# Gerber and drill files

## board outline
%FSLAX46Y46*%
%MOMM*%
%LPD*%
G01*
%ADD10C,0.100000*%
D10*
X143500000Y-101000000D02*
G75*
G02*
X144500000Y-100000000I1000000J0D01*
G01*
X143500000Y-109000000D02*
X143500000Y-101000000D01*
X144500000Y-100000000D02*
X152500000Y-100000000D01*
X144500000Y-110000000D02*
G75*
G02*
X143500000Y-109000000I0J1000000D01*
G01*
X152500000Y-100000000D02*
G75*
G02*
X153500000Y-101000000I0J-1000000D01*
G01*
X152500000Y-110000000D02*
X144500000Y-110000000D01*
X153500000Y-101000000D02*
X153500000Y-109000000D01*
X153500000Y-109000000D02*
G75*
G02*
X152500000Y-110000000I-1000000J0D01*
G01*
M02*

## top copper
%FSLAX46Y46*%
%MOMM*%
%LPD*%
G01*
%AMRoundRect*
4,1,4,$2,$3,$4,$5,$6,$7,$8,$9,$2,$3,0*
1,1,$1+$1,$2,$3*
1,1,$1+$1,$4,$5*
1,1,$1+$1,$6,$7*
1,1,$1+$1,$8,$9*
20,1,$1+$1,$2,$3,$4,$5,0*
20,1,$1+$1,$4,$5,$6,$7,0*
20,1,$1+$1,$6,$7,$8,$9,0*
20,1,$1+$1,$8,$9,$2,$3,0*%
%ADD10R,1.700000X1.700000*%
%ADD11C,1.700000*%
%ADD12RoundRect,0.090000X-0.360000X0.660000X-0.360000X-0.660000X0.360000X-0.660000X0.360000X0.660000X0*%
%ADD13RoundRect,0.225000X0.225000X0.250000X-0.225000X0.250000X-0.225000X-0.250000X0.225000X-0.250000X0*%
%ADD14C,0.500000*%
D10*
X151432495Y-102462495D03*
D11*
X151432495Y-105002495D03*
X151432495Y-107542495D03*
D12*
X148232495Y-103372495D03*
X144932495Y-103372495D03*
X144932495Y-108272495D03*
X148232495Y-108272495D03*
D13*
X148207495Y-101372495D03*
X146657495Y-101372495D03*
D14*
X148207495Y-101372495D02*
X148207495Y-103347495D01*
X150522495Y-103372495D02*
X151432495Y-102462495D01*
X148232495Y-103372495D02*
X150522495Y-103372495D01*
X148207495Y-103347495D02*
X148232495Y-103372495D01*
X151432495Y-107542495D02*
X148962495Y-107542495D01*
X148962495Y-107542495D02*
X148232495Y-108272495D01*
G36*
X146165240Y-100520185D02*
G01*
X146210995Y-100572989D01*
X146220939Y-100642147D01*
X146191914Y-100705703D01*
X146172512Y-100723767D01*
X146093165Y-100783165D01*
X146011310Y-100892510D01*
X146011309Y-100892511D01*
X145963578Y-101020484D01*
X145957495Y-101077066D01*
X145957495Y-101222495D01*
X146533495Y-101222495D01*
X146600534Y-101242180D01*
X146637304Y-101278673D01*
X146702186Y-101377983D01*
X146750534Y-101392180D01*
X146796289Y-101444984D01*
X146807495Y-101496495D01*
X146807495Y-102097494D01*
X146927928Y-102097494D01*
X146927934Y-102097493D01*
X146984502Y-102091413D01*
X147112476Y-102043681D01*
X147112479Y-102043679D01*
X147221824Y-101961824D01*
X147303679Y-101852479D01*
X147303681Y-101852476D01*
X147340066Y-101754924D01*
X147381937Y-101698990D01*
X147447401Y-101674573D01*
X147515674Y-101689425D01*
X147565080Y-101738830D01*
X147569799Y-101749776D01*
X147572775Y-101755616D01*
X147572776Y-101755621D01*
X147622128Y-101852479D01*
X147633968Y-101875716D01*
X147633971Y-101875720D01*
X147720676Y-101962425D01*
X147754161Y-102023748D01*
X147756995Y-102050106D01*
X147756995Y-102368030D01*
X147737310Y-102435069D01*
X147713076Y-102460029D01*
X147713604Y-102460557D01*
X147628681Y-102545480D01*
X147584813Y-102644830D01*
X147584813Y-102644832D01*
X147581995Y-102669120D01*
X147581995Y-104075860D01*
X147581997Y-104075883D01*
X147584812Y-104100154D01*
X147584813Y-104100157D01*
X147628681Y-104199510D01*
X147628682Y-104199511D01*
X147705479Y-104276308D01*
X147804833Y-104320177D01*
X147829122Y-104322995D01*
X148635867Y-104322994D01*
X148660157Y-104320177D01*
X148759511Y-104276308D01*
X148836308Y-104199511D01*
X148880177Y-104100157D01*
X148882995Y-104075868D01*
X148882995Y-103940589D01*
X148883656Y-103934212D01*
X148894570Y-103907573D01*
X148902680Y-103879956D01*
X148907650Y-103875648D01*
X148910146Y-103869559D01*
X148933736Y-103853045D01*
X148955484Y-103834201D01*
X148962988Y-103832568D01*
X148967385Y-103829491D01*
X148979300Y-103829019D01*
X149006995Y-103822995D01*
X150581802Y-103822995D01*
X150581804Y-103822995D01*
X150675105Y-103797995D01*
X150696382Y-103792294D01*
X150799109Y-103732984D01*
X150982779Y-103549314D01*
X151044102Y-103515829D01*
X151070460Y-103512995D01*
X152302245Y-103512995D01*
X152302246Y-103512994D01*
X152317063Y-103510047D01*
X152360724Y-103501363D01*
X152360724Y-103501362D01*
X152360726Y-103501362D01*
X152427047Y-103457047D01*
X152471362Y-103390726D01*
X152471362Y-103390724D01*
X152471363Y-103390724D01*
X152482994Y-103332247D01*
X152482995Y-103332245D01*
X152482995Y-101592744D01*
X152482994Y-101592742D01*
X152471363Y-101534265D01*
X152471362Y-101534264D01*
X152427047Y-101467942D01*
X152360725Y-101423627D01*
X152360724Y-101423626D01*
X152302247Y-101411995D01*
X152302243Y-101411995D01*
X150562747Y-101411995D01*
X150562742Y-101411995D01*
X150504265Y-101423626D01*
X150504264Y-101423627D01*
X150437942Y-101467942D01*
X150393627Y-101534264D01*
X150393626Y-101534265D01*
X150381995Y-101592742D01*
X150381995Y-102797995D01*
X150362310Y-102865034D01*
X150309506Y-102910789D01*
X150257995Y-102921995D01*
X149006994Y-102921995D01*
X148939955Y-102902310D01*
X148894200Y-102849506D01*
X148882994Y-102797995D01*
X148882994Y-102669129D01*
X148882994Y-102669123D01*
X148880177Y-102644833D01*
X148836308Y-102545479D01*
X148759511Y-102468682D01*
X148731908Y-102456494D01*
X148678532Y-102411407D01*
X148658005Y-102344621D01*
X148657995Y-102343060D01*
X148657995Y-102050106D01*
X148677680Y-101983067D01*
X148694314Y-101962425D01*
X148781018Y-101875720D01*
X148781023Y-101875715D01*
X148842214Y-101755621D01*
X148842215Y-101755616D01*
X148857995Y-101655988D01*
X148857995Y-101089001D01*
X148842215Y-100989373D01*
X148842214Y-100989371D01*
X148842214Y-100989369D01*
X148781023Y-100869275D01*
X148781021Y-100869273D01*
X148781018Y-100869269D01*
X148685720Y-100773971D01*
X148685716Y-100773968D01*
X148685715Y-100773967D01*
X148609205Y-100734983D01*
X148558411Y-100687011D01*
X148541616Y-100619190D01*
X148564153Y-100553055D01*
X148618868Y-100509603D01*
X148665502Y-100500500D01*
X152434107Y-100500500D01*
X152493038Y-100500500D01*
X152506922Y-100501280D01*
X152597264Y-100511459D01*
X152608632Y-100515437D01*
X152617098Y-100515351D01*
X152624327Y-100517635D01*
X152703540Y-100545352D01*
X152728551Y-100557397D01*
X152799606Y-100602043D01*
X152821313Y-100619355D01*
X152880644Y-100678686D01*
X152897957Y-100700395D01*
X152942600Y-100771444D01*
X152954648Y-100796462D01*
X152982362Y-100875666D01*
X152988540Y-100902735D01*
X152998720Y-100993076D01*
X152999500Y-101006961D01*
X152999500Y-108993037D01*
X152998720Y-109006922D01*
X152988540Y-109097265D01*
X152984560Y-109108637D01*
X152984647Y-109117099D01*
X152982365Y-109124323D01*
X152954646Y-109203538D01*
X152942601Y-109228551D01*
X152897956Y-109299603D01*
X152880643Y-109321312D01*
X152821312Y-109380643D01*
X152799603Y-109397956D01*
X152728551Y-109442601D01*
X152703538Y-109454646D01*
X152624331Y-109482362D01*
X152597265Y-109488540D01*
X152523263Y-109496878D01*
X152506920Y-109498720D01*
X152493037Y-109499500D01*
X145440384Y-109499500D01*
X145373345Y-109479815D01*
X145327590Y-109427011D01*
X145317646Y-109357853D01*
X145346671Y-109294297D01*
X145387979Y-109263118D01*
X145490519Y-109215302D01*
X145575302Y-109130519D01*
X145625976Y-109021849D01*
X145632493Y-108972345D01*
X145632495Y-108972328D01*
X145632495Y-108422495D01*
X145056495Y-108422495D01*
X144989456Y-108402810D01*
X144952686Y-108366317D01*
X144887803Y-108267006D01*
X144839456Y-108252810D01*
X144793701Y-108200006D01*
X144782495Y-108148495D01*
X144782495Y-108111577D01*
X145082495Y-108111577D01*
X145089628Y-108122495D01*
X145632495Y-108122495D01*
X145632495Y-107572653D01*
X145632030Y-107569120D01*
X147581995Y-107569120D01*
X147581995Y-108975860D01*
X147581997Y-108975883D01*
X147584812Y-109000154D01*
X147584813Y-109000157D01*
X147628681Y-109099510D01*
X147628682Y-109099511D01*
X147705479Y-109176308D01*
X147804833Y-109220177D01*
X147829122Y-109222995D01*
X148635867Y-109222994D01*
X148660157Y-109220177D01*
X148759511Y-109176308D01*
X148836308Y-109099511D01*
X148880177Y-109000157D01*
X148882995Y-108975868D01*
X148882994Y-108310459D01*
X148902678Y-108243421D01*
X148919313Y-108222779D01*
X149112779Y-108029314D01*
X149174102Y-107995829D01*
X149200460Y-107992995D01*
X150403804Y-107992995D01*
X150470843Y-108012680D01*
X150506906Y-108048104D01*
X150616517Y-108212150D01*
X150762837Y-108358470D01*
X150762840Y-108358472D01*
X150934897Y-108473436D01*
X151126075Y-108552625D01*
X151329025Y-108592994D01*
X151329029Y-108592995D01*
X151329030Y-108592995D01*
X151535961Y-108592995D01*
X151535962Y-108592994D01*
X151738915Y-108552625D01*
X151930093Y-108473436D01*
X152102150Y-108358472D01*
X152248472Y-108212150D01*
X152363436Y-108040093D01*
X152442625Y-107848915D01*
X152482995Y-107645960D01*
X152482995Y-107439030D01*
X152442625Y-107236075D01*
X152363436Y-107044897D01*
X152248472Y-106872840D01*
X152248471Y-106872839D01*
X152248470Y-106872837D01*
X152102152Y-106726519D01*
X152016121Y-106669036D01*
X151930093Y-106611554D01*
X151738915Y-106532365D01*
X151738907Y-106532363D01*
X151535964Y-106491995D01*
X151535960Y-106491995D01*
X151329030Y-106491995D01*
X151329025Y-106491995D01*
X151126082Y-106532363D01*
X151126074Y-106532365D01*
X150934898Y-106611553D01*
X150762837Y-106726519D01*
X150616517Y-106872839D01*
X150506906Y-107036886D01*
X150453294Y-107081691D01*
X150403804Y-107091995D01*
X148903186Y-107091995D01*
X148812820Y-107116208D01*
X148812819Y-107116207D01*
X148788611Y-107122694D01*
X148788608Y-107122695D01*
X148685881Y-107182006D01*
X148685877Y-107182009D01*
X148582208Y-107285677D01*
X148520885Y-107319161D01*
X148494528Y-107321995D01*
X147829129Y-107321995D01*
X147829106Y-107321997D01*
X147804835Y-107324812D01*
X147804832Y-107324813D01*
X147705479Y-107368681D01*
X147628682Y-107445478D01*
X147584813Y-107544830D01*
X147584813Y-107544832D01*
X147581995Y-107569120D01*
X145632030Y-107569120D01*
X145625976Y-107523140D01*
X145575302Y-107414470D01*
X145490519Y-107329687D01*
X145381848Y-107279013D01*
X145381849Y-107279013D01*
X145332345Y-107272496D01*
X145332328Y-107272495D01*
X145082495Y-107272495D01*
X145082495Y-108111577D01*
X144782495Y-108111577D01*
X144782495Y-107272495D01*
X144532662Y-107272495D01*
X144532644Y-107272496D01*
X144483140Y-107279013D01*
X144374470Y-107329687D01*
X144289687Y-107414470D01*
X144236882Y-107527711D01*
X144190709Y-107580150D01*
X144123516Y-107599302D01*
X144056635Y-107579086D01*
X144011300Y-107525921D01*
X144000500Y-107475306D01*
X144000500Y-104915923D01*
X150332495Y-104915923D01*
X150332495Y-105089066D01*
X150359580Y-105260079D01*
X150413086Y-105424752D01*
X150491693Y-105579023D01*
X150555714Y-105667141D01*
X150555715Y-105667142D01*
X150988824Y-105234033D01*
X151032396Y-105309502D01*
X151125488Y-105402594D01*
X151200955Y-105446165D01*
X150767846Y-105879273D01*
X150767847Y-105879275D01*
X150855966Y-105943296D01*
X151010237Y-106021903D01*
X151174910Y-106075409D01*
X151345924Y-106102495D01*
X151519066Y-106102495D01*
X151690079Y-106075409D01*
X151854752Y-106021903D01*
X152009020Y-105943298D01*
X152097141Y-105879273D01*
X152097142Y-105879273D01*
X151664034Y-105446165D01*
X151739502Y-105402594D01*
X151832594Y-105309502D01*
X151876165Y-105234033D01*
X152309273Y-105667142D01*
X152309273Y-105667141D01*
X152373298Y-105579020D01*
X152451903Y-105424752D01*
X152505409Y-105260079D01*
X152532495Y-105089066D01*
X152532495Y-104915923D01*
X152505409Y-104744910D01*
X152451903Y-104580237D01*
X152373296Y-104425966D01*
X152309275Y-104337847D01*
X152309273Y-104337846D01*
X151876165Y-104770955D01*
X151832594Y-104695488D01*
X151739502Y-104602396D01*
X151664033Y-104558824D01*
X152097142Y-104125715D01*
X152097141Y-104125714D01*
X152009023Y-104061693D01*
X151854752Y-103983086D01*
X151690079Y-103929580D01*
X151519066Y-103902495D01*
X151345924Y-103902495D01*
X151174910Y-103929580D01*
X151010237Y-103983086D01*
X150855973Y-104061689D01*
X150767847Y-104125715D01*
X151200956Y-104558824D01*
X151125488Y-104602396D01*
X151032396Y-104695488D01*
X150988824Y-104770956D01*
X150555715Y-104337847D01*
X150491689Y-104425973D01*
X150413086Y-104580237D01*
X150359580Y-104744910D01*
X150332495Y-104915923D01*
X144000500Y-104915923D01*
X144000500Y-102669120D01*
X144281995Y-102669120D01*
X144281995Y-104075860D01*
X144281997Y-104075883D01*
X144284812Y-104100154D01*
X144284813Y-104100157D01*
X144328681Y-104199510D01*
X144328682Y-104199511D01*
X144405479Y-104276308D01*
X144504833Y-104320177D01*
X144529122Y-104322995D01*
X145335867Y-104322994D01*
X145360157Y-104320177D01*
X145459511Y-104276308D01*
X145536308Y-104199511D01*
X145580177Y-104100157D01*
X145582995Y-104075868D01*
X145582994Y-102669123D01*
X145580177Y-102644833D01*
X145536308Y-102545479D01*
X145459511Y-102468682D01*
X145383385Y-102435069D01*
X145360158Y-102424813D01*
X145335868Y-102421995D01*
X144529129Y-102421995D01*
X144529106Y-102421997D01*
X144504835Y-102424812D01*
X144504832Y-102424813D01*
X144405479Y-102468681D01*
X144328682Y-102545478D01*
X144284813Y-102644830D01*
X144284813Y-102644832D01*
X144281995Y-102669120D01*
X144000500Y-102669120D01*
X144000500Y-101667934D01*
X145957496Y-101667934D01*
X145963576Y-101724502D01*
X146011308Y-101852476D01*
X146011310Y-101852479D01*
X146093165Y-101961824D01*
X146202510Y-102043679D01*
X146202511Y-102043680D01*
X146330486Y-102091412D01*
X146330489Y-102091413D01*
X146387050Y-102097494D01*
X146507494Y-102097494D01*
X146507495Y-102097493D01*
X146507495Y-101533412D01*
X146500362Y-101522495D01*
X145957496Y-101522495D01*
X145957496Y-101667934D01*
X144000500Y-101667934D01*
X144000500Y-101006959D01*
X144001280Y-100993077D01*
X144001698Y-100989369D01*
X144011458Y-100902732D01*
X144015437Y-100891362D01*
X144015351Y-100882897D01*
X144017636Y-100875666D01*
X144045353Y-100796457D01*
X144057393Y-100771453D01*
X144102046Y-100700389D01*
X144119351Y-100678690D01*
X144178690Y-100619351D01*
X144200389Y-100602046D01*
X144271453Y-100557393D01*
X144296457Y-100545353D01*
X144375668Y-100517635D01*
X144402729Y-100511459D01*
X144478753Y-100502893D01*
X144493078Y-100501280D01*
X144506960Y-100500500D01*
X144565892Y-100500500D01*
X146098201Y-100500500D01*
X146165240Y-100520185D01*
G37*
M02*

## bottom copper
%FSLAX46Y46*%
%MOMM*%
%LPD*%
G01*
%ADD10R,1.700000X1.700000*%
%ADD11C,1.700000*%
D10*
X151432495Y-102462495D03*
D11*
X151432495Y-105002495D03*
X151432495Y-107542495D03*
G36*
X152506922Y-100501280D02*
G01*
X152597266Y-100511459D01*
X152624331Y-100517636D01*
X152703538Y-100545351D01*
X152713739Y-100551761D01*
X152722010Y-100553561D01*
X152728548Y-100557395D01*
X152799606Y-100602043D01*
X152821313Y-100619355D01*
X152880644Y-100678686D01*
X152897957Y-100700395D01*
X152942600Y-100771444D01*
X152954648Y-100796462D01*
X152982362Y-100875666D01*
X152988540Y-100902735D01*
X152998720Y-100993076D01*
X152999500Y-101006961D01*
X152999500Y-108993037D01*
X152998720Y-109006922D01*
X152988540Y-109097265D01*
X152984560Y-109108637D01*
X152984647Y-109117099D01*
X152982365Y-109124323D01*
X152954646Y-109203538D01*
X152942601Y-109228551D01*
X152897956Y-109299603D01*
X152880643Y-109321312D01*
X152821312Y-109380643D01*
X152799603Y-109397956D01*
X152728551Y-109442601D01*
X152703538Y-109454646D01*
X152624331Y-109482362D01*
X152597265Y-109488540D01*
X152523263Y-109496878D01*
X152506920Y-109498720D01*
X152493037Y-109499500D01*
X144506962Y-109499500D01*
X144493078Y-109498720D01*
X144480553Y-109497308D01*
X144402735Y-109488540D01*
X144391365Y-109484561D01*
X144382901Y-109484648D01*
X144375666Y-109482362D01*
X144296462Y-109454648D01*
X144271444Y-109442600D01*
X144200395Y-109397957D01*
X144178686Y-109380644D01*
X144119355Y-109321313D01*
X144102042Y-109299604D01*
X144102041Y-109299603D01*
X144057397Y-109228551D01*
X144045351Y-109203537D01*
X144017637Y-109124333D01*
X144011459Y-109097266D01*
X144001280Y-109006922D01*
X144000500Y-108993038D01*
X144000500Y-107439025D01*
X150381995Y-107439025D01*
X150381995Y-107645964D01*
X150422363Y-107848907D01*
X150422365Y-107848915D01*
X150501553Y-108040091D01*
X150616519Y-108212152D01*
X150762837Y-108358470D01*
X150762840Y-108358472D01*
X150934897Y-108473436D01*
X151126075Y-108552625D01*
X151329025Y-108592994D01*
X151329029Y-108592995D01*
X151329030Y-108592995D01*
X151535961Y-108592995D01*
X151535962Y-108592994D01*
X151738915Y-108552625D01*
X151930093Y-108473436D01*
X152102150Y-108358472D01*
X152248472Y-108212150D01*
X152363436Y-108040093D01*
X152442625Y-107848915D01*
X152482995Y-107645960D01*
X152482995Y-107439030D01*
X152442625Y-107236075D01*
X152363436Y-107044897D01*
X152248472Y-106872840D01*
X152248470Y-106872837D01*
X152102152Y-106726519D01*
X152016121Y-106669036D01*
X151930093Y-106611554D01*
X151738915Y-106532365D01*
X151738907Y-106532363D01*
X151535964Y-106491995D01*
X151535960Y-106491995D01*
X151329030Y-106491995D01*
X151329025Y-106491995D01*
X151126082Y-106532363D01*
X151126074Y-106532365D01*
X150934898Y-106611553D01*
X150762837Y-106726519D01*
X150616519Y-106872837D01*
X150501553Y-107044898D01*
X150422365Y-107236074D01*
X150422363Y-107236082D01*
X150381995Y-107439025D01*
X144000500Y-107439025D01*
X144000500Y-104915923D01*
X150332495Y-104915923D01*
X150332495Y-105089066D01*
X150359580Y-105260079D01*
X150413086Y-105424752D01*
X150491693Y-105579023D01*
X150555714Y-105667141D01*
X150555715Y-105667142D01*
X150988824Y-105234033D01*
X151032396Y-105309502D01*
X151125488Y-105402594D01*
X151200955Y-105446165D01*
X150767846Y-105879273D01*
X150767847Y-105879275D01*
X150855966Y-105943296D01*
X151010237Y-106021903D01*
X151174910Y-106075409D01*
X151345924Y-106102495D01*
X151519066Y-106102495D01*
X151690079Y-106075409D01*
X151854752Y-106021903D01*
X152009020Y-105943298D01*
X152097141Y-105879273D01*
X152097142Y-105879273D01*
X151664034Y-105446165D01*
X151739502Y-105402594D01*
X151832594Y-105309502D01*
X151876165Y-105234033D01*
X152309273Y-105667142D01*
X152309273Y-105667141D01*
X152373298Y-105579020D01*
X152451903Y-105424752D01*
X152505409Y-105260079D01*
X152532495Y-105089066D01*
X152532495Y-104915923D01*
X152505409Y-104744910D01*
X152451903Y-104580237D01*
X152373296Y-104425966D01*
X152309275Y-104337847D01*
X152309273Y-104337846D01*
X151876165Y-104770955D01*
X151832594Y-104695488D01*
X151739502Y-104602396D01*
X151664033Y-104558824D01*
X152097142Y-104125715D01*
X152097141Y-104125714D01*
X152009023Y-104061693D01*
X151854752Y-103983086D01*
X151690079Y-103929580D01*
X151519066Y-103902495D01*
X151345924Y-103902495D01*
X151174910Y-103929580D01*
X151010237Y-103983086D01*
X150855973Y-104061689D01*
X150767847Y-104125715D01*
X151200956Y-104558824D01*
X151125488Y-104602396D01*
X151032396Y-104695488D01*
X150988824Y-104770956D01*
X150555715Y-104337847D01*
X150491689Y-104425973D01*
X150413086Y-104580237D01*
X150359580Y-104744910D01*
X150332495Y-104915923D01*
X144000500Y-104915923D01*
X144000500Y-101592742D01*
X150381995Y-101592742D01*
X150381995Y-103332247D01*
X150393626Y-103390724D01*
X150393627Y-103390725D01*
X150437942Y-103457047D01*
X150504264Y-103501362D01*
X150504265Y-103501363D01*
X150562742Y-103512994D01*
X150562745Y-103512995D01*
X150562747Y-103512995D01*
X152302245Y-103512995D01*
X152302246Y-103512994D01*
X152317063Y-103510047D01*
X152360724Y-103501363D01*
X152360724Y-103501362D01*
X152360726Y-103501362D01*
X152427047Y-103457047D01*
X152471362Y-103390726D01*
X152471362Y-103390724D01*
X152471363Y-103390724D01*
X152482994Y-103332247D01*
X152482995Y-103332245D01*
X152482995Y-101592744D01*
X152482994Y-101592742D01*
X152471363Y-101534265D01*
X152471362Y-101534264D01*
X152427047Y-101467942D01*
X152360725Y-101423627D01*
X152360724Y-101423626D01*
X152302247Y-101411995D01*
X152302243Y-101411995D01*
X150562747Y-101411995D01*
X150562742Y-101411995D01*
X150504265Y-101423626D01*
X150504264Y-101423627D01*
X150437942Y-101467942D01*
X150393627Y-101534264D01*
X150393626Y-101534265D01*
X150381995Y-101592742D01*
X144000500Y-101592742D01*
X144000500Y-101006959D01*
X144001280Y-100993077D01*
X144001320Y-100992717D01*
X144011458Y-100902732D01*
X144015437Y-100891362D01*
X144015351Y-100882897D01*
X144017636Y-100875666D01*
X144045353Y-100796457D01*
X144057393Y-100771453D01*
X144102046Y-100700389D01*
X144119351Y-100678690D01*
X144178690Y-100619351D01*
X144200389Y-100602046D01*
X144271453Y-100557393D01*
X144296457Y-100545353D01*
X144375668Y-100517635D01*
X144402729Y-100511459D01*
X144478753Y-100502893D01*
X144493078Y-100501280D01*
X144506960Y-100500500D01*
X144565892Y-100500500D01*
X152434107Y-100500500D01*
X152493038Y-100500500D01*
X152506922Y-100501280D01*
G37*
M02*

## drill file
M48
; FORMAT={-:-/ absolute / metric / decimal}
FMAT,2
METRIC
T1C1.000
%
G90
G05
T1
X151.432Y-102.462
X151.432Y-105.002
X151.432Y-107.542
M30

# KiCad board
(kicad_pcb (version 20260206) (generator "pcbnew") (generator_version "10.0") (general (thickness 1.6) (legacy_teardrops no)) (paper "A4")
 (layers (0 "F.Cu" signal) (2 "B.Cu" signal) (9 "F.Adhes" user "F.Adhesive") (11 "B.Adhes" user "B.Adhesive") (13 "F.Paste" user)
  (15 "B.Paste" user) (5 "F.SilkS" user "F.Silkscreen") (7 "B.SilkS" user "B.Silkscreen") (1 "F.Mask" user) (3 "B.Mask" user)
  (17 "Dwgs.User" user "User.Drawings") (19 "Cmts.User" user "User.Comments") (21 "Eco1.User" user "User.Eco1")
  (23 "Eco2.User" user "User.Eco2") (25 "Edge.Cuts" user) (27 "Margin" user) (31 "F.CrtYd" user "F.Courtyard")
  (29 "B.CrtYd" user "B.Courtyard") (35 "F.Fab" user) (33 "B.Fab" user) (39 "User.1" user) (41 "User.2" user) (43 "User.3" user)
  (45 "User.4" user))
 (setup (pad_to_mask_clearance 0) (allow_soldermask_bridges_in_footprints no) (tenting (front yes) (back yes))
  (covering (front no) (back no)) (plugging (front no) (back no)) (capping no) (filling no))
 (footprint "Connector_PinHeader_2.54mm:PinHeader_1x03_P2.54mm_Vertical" (layer "F.Cu") (at 151.432495 102.462495)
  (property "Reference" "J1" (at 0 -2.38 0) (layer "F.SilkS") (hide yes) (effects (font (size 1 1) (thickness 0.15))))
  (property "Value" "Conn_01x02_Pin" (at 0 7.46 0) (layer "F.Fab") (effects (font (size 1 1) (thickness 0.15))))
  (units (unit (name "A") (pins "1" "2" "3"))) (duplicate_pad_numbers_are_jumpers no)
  (pad "1" thru_hole rect (at 0 0) (size 1.7 1.7) (drill 1) (layers "*.Cu" "*.Mask") (remove_unused_layers no) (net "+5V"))
  (pad "2" thru_hole circle (at 0 2.54) (size 1.7 1.7) (drill 1) (layers "*.Cu" "*.Mask") (remove_unused_layers no) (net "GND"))
  (pad "3" thru_hole circle (at 0 5.08) (size 1.7 1.7) (drill 1) (layers "*.Cu" "*.Mask") (remove_unused_layers no) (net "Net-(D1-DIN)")))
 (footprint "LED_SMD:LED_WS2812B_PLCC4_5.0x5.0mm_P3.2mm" (layer "F.Cu") (at 146.582495 105.822495 -90)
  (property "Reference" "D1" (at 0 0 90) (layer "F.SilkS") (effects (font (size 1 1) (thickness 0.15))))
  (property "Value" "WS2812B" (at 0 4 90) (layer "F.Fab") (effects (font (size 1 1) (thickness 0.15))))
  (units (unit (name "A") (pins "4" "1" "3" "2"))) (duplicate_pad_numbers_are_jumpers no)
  (pad "1" smd roundrect (at -2.45 -1.65 270) (size 1.5 0.9) (layers "F.Cu" "F.Mask" "F.Paste") (roundrect_rratio 0.1) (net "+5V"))
  (pad "2" smd roundrect (at -2.45 1.65 270) (size 1.5 0.9) (layers "F.Cu" "F.Mask" "F.Paste") (roundrect_rratio 0.1)
   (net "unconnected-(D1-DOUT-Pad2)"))
  (pad "3" smd roundrect (at 2.45 1.65 270) (size 1.5 0.9) (layers "F.Cu" "F.Mask" "F.Paste") (roundrect_rratio 0.1) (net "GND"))
  (pad "4" smd roundrect (at 2.45 -1.65 270) (size 1.5 0.9) (layers "F.Cu" "F.Mask" "F.Paste") (roundrect_rratio 0.1) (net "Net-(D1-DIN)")))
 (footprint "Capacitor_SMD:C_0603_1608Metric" (layer "F.Cu") (at 147.432495 101.372495 180)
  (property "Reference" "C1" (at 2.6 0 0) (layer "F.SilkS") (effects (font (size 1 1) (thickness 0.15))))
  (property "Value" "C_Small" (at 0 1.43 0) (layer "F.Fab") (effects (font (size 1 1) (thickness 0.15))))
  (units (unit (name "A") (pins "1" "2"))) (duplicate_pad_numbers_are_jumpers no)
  (pad "1" smd roundrect (at -0.775 0 180) (size 0.9 0.95) (layers "F.Cu" "F.Mask" "F.Paste") (roundrect_rratio 0.25) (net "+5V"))
  (pad "2" smd roundrect (at 0.775 0 180) (size 0.9 0.95) (layers "F.Cu" "F.Mask" "F.Paste") (roundrect_rratio 0.25) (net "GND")))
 (gr_arc (start 143.5 101) (mid 143.792893 100.292893) (end 144.5 100) (stroke (width 0.1) (type default)) (layer "Edge.Cuts"))
 (gr_line (start 143.5 109) (end 143.5 101) (stroke (width 0.1) (type default)) (layer "Edge.Cuts"))
 (gr_line (start 144.5 100) (end 152.5 100) (stroke (width 0.1) (type default)) (layer "Edge.Cuts"))
 (gr_arc (start 144.5 110) (mid 143.792893 109.707106) (end 143.5 109) (stroke (width 0.1) (type default)) (layer "Edge.Cuts"))
 (gr_arc (start 152.5 100) (mid 153.207106 100.292893) (end 153.5 101) (stroke (width 0.1) (type default)) (layer "Edge.Cuts"))
 (gr_line (start 152.5 110) (end 144.5 110) (stroke (width 0.1) (type default)) (layer "Edge.Cuts"))
 (gr_line (start 153.5 101) (end 153.5 109) (stroke (width 0.1) (type default)) (layer "Edge.Cuts"))
 (gr_arc (start 153.5 109) (mid 153.207106 109.707106) (end 152.5 110) (stroke (width 0.1) (type default)) (layer "Edge.Cuts"))
 (segment (start 148.207495 101.372495) (end 148.207495 103.347495) (width 0.5) (layer "F.Cu") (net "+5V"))
 (segment (start 150.522495 103.372495) (end 151.432495 102.462495) (width 0.5) (layer "F.Cu") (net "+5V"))
 (segment (start 148.232495 103.372495) (end 150.522495 103.372495) (width 0.5) (layer "F.Cu") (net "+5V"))
 (segment (start 148.207495 103.347495) (end 148.232495 103.372495) (width 0.5) (layer "F.Cu") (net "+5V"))
 (segment (start 151.432495 107.542495) (end 148.962495 107.542495) (width 0.5) (layer "F.Cu") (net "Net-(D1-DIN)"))
 (segment (start 148.962495 107.542495) (end 148.232495 108.272495) (width 0.5) (layer "F.Cu") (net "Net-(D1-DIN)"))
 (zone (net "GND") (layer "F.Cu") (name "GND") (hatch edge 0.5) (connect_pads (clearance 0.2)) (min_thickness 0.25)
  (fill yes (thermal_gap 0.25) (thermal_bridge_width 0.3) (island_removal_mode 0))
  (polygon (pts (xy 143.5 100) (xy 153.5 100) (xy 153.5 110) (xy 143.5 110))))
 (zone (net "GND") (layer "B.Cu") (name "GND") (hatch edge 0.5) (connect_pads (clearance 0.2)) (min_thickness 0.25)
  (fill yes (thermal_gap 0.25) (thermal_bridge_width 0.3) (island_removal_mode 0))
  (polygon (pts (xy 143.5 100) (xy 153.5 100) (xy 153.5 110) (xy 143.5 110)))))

